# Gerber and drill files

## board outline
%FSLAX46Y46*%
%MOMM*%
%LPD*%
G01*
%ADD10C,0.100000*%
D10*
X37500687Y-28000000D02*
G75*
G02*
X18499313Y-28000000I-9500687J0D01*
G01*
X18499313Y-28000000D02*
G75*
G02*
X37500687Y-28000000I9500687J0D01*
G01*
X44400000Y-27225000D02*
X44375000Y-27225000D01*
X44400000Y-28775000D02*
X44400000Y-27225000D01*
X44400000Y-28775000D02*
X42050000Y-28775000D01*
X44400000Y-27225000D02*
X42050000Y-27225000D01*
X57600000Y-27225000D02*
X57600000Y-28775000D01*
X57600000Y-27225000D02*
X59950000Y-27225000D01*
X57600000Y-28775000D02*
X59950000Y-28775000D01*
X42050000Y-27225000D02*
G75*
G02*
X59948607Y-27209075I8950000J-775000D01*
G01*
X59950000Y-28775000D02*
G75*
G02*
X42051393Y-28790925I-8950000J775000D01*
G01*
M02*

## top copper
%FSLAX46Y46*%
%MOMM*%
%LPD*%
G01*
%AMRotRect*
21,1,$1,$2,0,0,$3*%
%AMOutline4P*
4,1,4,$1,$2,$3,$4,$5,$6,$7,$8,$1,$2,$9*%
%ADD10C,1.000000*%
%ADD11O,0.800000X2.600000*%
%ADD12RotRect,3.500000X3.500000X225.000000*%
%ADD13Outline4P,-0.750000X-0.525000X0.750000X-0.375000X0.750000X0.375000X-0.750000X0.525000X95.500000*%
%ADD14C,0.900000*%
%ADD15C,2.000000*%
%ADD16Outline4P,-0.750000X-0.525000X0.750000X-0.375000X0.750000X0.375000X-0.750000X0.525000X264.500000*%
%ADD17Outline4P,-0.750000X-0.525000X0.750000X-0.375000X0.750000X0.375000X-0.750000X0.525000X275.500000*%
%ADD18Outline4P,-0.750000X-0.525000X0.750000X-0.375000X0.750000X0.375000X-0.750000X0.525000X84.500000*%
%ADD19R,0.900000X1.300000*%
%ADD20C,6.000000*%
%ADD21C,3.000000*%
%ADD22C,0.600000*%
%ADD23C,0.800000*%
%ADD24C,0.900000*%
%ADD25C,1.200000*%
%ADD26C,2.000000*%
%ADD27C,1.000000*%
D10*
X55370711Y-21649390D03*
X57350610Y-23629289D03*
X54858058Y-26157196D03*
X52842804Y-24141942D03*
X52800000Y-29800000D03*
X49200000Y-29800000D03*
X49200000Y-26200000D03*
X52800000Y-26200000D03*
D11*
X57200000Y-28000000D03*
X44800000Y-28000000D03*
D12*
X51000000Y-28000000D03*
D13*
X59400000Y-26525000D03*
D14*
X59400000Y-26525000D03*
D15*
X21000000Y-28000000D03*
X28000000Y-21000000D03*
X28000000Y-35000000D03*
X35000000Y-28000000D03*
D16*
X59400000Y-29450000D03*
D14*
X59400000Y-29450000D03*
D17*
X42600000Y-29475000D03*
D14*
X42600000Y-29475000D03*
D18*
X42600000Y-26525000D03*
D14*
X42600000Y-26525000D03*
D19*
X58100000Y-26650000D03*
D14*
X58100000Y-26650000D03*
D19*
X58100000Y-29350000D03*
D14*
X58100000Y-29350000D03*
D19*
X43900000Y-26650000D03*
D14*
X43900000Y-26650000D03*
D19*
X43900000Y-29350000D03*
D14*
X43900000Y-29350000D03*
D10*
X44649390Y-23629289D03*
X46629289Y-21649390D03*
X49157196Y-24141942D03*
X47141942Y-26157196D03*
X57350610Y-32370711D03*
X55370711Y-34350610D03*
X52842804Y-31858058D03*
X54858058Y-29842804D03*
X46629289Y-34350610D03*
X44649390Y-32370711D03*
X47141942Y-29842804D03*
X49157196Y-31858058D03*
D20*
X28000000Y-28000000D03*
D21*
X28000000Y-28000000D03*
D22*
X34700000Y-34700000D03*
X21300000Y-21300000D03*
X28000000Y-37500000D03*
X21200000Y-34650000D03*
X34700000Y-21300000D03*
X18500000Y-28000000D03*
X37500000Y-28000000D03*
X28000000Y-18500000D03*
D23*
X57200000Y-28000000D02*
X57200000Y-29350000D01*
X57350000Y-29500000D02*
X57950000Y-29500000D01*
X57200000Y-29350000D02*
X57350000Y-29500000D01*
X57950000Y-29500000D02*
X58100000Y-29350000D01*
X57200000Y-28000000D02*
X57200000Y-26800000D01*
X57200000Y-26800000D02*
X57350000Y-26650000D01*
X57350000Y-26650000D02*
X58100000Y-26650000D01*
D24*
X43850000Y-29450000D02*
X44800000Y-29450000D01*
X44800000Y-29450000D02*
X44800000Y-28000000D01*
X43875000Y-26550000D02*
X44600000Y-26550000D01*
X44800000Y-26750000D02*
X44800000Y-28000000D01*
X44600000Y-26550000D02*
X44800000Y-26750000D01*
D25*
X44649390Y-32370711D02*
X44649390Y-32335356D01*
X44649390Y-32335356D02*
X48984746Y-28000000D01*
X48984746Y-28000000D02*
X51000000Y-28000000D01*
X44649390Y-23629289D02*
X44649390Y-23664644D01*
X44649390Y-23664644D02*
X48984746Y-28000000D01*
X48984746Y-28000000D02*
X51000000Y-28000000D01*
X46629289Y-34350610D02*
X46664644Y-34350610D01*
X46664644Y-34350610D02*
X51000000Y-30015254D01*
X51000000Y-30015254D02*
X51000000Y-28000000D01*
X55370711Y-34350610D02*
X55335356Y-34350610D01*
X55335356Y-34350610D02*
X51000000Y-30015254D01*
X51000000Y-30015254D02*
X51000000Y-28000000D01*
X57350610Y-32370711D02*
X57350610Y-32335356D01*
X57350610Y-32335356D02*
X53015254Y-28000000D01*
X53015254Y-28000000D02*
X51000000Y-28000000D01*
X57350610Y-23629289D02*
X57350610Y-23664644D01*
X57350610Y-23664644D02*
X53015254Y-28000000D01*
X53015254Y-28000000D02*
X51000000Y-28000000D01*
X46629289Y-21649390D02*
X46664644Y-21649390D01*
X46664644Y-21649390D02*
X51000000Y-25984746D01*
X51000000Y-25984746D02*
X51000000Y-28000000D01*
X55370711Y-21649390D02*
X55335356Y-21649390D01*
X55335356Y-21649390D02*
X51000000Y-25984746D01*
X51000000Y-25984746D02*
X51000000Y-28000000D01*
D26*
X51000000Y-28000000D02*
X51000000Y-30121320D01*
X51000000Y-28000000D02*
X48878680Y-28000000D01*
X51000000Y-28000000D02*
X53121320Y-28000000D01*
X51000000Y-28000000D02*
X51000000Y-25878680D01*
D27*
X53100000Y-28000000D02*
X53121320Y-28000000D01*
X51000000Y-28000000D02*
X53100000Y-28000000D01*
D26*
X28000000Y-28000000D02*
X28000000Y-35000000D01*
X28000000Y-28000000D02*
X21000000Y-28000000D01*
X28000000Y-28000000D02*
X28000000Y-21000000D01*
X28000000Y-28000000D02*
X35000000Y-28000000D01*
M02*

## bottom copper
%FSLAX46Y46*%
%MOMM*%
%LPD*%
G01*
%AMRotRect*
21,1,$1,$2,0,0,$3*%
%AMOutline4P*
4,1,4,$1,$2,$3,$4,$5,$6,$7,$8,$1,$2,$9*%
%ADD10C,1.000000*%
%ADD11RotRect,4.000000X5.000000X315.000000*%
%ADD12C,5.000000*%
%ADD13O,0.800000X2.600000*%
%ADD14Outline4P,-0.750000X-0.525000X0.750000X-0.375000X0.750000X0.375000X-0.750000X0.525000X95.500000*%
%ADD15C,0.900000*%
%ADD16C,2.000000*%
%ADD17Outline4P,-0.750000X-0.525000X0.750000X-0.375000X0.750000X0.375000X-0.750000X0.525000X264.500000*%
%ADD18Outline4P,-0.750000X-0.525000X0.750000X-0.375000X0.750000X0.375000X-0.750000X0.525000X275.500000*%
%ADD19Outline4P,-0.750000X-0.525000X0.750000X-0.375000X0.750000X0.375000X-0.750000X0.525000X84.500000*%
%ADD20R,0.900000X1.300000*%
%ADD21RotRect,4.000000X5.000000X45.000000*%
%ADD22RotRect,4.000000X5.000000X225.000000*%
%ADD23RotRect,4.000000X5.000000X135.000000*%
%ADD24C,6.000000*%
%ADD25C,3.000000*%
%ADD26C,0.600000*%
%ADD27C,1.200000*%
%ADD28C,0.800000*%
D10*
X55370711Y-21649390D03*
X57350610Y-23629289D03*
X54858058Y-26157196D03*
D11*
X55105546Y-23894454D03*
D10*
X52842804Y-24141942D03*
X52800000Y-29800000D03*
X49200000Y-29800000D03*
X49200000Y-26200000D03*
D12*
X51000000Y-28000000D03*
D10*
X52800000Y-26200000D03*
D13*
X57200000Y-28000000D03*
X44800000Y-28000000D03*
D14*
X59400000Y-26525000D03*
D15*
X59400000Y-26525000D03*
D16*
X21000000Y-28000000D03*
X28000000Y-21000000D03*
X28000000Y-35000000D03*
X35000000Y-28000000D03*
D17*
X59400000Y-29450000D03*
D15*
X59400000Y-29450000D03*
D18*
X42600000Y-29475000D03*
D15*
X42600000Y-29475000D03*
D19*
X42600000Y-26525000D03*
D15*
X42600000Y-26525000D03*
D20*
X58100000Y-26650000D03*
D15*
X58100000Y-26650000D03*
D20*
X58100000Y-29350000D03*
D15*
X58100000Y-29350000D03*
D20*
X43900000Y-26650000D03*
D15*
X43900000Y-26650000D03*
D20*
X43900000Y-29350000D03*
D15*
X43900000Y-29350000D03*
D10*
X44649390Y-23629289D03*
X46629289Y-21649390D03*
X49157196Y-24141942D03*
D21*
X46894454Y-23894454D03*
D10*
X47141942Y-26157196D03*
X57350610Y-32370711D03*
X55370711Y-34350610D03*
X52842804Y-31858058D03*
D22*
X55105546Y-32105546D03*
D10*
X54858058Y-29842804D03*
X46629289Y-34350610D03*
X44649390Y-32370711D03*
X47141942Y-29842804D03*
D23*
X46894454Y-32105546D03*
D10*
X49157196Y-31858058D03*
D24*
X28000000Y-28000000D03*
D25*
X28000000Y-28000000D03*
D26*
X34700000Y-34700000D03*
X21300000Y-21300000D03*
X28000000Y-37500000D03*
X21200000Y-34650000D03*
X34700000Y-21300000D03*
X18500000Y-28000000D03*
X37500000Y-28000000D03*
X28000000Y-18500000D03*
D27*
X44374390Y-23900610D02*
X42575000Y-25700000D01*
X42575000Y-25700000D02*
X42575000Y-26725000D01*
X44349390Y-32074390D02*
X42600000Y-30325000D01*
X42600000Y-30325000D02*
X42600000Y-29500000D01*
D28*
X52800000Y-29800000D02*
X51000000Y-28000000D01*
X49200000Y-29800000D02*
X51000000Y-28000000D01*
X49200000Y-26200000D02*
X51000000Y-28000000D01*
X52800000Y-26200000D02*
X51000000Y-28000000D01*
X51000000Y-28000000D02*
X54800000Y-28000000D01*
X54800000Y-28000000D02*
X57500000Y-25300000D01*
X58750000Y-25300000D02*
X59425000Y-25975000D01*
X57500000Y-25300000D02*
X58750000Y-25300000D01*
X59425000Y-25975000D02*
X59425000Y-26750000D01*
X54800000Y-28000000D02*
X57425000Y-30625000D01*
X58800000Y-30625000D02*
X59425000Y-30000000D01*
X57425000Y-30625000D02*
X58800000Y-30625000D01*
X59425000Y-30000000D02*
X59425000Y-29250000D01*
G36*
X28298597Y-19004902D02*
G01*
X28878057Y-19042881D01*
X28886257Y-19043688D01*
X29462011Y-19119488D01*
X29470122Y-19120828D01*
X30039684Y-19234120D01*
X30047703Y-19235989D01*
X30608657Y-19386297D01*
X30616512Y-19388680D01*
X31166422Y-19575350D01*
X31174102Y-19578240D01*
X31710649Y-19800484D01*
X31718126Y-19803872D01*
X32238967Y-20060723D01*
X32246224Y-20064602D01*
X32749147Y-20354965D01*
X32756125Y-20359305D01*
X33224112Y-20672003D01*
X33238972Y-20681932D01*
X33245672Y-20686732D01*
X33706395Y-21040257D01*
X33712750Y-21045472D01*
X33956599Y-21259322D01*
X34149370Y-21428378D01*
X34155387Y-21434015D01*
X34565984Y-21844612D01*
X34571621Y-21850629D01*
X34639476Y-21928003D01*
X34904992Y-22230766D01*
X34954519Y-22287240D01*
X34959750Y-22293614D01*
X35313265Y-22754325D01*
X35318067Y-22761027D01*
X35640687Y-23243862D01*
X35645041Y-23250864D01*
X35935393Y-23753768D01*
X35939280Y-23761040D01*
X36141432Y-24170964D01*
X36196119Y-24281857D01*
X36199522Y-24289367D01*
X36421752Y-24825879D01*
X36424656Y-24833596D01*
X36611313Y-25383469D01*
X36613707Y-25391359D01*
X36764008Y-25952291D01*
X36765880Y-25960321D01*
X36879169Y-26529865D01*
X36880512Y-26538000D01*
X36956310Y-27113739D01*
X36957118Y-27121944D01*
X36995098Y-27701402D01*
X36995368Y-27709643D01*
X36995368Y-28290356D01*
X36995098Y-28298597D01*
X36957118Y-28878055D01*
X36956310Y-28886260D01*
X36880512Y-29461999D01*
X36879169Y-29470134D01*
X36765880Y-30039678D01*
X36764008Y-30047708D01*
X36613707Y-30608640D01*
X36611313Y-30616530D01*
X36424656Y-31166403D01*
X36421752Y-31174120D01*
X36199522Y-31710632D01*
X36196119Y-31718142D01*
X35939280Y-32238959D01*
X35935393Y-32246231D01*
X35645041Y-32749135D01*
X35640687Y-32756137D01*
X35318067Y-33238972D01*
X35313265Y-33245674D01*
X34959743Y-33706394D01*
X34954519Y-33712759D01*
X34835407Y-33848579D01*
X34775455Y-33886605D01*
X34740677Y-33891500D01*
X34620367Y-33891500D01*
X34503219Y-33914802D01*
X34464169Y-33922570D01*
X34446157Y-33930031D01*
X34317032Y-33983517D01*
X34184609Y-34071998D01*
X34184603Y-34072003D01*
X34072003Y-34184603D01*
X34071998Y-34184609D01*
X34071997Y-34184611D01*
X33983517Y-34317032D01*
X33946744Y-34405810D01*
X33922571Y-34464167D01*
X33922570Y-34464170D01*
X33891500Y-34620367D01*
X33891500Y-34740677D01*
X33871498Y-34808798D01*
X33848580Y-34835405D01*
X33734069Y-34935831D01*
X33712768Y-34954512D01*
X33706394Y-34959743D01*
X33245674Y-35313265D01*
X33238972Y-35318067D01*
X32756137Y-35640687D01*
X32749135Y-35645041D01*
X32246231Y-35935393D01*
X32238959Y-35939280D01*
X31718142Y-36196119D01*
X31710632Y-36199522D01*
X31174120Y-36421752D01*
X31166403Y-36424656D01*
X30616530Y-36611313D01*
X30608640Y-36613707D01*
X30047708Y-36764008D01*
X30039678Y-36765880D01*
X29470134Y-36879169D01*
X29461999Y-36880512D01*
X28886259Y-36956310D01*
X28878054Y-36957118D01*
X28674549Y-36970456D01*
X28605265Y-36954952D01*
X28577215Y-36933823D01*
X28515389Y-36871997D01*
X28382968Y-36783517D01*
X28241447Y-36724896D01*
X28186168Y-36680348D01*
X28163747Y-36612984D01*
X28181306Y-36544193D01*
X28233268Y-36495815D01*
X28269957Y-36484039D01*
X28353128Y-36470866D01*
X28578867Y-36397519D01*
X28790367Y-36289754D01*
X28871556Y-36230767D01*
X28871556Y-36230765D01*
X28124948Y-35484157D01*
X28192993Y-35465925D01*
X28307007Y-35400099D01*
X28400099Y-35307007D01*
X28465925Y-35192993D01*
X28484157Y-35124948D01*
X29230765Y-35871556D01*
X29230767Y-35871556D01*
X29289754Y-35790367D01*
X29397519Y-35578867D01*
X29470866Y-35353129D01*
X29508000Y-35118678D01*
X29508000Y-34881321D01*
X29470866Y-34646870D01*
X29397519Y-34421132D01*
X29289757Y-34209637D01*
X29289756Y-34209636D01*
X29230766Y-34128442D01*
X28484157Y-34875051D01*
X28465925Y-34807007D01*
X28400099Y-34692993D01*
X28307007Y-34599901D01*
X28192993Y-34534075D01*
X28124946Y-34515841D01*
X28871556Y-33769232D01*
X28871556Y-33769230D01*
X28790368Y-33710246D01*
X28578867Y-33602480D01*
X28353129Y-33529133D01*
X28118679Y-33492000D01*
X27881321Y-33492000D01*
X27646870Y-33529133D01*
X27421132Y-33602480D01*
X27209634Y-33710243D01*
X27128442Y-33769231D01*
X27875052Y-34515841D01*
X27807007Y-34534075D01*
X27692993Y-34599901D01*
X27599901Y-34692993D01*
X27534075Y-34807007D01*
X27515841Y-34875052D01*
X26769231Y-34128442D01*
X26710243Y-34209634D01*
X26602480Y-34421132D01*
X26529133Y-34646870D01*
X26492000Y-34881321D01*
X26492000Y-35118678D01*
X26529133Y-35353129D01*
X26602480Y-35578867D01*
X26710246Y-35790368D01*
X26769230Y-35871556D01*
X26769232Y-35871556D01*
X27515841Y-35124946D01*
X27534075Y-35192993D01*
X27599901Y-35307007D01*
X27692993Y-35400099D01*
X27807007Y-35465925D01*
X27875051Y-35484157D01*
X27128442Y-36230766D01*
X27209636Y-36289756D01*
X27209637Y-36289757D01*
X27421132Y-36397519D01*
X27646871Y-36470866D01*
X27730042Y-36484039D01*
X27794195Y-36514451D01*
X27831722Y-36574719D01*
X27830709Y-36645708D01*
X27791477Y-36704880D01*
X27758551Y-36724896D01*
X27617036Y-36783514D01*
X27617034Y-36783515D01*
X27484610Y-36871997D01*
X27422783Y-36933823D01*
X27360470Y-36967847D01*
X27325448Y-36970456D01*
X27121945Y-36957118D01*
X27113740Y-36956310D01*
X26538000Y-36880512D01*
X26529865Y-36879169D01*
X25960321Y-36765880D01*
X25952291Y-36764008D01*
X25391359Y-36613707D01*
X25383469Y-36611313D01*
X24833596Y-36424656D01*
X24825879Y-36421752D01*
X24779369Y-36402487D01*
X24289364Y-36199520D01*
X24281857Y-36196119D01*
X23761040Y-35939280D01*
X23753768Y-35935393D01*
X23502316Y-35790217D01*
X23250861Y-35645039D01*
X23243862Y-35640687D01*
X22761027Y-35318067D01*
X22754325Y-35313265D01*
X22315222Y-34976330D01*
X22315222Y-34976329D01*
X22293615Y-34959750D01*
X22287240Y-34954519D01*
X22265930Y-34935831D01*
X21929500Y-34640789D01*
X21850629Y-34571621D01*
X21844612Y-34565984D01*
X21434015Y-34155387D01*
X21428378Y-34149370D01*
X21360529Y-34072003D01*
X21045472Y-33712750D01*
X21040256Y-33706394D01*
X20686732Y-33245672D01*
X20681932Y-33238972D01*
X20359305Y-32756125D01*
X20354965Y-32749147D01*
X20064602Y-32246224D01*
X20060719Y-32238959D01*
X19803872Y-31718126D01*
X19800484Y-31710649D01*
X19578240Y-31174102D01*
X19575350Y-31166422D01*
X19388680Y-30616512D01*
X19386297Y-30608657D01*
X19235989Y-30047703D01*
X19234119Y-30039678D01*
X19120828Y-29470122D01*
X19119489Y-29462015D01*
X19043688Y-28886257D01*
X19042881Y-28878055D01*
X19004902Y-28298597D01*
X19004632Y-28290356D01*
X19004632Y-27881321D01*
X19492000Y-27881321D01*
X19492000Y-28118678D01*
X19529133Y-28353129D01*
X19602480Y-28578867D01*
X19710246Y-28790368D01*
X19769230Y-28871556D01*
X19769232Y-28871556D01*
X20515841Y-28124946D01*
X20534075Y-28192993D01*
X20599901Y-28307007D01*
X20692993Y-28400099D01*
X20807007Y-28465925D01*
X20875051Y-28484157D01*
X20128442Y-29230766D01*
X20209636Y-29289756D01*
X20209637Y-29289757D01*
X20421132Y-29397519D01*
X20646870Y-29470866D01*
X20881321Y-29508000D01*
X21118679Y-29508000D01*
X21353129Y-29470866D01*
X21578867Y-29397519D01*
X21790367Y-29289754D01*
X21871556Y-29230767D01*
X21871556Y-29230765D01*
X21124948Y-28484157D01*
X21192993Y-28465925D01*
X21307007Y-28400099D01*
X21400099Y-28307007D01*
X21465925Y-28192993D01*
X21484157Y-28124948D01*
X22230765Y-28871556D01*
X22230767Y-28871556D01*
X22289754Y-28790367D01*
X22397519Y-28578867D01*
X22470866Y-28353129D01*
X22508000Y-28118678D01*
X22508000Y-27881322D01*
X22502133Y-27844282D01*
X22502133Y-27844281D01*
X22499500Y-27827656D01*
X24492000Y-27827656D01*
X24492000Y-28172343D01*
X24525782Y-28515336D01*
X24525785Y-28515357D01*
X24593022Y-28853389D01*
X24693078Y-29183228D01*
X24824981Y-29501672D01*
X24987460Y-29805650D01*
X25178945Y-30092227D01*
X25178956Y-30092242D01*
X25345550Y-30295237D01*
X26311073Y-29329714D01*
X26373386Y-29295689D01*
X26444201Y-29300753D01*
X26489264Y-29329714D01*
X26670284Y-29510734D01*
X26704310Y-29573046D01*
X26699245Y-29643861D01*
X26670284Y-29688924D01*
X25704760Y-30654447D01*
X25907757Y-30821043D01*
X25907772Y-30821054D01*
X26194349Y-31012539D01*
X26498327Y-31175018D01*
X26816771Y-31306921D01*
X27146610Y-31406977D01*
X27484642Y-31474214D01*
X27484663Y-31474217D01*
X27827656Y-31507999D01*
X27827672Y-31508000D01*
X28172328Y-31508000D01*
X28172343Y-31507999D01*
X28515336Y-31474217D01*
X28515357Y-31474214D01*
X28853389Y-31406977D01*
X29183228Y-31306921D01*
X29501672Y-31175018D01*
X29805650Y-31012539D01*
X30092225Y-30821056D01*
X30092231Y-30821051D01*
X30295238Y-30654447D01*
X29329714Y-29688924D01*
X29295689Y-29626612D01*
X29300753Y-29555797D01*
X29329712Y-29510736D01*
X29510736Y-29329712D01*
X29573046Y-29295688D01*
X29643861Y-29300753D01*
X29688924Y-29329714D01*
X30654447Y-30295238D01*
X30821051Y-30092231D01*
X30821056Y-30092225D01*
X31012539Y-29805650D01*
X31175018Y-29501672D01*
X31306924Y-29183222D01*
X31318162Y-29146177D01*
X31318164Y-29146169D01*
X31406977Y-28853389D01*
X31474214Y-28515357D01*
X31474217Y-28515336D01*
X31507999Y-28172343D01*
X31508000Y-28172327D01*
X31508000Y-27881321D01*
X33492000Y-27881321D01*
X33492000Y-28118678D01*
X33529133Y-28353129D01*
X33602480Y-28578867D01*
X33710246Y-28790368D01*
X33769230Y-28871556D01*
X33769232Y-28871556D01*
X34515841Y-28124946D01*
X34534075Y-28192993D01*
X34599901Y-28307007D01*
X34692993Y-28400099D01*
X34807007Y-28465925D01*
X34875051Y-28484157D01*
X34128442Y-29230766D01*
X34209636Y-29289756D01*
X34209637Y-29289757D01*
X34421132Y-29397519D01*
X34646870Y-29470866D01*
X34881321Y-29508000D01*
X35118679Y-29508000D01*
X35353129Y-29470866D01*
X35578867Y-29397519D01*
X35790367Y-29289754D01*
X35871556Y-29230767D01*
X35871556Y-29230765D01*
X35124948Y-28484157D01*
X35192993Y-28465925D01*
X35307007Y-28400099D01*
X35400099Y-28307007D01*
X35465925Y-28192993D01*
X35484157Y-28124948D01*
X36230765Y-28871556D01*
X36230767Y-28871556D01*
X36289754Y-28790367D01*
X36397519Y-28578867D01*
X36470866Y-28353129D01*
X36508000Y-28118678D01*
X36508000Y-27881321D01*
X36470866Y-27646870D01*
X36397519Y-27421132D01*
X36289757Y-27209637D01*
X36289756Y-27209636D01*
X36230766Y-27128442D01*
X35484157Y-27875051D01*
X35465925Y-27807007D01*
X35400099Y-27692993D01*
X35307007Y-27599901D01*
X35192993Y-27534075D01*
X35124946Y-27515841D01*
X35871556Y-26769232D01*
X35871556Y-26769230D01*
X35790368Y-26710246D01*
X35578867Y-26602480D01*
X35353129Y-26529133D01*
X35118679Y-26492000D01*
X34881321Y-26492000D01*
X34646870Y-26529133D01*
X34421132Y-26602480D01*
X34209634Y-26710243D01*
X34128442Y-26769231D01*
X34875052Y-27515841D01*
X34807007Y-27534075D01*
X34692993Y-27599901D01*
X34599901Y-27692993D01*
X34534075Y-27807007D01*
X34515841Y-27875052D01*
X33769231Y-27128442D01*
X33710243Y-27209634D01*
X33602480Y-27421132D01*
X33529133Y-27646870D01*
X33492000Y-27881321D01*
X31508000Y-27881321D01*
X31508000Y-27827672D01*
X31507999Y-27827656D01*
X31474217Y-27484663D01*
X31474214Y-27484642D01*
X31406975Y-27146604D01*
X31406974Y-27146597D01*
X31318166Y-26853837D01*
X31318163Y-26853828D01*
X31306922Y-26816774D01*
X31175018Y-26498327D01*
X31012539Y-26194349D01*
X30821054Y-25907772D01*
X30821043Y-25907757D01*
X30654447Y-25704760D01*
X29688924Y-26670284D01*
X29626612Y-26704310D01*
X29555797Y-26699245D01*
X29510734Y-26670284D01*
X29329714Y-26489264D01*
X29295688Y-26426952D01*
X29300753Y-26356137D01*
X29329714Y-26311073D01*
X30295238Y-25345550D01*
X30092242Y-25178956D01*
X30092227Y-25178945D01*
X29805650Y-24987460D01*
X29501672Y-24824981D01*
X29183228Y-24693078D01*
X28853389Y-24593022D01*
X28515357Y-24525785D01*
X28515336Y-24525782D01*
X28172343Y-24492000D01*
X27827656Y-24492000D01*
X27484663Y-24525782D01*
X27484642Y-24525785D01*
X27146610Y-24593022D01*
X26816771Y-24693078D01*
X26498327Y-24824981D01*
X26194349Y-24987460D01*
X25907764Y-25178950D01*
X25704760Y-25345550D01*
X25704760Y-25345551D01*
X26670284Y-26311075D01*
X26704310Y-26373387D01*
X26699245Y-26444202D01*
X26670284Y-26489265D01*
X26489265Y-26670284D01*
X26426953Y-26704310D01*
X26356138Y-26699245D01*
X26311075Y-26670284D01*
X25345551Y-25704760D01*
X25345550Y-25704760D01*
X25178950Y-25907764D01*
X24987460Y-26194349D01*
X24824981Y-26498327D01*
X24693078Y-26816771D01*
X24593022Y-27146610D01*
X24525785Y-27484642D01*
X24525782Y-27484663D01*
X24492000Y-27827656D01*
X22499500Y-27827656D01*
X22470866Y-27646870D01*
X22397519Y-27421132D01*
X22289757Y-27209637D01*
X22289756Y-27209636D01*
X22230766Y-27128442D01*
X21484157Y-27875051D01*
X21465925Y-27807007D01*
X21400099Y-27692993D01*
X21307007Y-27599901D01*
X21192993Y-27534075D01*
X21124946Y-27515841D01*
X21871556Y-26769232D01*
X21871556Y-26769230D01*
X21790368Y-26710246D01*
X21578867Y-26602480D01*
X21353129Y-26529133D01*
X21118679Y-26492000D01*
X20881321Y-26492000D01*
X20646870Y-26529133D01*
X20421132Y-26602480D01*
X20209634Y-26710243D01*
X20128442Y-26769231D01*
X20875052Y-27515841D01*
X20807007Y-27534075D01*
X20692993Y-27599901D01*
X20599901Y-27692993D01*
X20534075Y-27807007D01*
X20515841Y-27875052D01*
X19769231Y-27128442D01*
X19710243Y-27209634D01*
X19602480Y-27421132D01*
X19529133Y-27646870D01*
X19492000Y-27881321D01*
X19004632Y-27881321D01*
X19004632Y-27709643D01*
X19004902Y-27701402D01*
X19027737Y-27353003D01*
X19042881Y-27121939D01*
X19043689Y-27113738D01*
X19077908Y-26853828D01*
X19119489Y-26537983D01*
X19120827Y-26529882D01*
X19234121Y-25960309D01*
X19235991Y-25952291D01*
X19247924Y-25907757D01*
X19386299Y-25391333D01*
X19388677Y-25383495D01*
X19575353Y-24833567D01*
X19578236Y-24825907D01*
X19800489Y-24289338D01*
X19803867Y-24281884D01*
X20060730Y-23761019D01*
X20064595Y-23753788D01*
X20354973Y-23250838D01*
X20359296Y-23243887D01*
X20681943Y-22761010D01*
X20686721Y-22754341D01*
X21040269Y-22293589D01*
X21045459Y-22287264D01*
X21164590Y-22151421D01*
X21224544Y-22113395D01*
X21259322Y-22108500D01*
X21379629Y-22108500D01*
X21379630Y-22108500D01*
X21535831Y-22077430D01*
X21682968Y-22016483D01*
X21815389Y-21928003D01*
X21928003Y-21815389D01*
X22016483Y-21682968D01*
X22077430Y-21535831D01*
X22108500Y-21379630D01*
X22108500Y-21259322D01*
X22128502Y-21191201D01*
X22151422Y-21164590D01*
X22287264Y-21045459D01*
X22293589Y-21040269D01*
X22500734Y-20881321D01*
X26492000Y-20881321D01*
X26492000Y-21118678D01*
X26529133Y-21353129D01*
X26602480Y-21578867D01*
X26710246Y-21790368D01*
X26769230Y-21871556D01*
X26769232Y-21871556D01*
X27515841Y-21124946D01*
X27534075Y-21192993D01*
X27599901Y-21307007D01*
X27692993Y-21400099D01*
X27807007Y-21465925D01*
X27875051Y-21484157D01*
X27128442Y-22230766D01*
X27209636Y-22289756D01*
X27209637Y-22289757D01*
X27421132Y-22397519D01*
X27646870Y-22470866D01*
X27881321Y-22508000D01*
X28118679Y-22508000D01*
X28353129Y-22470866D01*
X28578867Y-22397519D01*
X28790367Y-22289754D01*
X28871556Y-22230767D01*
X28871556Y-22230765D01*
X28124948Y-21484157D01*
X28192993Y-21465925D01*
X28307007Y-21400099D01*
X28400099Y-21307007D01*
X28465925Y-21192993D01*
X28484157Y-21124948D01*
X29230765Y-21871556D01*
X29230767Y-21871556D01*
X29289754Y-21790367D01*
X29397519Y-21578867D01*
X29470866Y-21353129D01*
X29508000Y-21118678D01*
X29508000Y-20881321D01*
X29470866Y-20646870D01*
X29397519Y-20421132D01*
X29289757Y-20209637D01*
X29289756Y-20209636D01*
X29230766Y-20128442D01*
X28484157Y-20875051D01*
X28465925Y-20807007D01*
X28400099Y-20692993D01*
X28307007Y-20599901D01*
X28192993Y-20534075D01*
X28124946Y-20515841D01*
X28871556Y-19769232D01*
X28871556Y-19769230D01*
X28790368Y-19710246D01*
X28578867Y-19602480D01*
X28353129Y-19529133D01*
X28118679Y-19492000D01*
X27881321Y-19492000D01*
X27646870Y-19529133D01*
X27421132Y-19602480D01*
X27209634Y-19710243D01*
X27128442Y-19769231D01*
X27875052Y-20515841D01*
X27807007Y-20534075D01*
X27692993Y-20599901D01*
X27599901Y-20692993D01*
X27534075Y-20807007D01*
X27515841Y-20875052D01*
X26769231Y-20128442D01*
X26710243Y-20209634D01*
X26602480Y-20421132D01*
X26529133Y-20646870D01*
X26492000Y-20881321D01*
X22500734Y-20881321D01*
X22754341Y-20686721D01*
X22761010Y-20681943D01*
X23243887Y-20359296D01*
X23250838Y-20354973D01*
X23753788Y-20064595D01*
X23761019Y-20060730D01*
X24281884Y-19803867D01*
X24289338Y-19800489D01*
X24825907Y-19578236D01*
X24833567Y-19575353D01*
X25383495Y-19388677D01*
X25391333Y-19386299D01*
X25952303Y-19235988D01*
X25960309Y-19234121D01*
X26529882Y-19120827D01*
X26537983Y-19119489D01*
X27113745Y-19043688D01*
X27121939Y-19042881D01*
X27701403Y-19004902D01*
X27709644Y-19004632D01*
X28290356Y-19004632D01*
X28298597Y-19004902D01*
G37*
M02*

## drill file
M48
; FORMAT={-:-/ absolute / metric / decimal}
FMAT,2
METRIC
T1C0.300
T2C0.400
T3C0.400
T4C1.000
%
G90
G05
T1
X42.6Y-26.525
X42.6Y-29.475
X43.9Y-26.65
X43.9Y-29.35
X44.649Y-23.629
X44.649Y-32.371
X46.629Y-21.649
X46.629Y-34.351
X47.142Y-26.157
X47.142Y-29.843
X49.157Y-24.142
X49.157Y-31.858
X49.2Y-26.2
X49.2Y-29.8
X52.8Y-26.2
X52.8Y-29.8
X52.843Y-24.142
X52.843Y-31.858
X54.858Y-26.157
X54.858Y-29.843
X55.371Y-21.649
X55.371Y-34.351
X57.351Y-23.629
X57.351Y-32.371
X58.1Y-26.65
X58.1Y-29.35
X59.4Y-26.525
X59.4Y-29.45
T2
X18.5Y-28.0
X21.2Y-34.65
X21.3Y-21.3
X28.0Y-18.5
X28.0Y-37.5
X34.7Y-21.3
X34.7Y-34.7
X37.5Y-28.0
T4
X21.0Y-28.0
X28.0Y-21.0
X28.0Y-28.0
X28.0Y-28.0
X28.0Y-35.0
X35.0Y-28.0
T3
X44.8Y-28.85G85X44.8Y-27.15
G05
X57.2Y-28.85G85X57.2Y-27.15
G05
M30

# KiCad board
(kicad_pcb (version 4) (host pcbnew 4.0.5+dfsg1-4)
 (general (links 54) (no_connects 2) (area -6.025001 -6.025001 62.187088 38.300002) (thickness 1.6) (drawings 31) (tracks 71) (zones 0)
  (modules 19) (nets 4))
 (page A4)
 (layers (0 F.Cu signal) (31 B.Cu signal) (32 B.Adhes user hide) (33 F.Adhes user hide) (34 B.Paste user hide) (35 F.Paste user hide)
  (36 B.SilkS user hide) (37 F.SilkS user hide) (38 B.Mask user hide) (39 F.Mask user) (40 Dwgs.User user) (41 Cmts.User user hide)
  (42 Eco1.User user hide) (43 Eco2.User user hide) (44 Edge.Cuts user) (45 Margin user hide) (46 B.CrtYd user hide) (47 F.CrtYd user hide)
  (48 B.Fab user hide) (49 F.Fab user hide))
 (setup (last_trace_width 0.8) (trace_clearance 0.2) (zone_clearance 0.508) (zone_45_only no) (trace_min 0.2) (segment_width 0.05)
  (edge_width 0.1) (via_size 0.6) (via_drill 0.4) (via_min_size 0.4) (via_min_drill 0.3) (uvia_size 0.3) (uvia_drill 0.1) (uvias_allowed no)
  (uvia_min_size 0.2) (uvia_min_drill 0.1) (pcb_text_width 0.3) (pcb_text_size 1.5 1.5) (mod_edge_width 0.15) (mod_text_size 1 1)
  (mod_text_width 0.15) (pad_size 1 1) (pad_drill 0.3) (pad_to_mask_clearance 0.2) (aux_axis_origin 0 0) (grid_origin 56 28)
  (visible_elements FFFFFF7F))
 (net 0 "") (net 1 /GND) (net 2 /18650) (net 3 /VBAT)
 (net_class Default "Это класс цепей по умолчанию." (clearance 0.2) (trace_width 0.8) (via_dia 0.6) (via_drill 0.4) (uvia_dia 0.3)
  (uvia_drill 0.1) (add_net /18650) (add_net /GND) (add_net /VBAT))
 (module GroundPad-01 (layer F.Cu) (at 55.3 23.7 315)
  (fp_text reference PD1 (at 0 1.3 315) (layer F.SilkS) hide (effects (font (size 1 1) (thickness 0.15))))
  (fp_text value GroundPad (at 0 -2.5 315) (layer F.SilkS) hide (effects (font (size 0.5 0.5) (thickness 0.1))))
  (pad 2 thru_hole circle (at -1.4 -1.5 315) (size 1 1) (drill 0.3) (layers *.Cu) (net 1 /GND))
  (pad 3 thru_hole circle (at 1.4 -1.5 315) (size 1 1) (drill 0.3) (layers *.Cu) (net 1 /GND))
  (pad 5 thru_hole circle (at 1.425 2.05 315) (size 1 1) (drill 0.3) (layers *.Cu) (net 1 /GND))
  (pad 1 smd rect (at 0 0.275 315) (size 4 5) (layers B.Cu B.Paste B.Mask) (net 1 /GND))
  (pad 4 thru_hole circle (at -1.425 2.05 315) (size 1 1) (drill 0.3) (layers *.Cu) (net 1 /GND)))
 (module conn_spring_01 (layer B.Cu) (at 51 28 270)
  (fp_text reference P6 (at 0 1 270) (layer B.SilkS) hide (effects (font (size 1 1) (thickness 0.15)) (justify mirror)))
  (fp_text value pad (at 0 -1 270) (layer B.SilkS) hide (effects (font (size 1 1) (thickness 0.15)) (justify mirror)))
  (pad 4 thru_hole circle (at 1.8 -1.8 270) (size 1 1) (drill 0.3) (layers *.Cu) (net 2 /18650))
  (pad 3 thru_hole circle (at 1.8 1.8 270) (size 1 1) (drill 0.3) (layers *.Cu) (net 2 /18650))
  (pad 2 thru_hole circle (at -1.8 1.8 270) (size 1 1) (drill 0.3) (layers *.Cu) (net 2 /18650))
  (pad 1 smd circle (at 0 0 270) (size 5 5) (layers B.Cu B.Paste B.Mask) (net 2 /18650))
  (pad 5 thru_hole circle (at -1.8 -1.8 270) (size 1 1) (drill 0.3) (layers *.Cu) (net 2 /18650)))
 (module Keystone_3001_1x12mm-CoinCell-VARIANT (layer F.Cu) (at 51 28 180)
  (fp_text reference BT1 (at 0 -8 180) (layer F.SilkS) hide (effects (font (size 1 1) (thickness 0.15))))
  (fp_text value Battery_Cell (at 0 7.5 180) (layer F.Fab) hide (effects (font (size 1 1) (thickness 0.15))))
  (pad 1 thru_hole oval (at -6.2 0 180) (size 0.8 2.6) (drill oval 0.4 2.1) (layers *.Cu *.Mask) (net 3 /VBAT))
  (pad 1 thru_hole oval (at 6.2 0 180) (size 0.8 2.6) (drill oval 0.4 2.1) (layers *.Cu *.Mask) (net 3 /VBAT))
  (pad 2 smd rect (at 0 0 225) (size 3.5 3.5) (layers F.Cu F.Mask) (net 1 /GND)))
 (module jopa (layer F.Cu) (at 59.4 26.525 95.5)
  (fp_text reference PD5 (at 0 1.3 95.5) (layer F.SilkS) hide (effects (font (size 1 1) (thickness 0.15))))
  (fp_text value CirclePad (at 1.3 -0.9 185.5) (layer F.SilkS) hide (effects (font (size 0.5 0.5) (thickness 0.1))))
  (pad 1 smd trapezoid (at 0 0 95.5) (size 1.5 0.9) (rect_delta 0.15 0) (layers F.Cu F.Paste F.Mask) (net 2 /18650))
  (pad 2 smd trapezoid (at 0 0 95.5) (size 1.5 0.9) (rect_delta 0.15 0) (layers B.Cu F.Paste B.Mask) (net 2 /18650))
  (pad 3 thru_hole circle (at 0 0 95.5) (size 0.9 0.9) (drill 0.3) (layers *.Cu *.Mask) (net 2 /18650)))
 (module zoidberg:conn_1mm (layer F.Cu) (at 21 28)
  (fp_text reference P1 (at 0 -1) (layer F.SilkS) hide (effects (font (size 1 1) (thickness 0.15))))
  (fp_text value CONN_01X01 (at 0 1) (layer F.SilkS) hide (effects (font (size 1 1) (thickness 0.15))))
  (pad 1 thru_hole circle (at 0 0) (size 2 2) (drill 1) (layers *.Cu) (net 1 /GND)))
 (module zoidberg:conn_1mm (layer F.Cu) (at 28 21)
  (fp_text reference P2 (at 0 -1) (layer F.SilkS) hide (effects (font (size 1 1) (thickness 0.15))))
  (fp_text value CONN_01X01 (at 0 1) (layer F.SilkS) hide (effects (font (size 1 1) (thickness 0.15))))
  (pad 1 thru_hole circle (at 0 0) (size 2 2) (drill 1) (layers *.Cu) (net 1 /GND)))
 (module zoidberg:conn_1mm (layer F.Cu) (at 28 35)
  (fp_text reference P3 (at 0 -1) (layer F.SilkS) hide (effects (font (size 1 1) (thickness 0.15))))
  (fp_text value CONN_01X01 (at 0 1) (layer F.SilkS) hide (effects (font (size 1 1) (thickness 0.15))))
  (pad 1 thru_hole circle (at 0 0) (size 2 2) (drill 1) (layers *.Cu) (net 1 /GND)))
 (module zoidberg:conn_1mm (layer F.Cu) (at 35 28)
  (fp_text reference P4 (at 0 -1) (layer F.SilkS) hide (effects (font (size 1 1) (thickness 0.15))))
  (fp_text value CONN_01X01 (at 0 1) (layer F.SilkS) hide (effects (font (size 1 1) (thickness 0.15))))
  (pad 1 thru_hole circle (at 0 0) (size 2 2) (drill 1) (layers *.Cu) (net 1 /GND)))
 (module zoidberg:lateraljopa (layer F.Cu) (at 59.4 29.45 264.5)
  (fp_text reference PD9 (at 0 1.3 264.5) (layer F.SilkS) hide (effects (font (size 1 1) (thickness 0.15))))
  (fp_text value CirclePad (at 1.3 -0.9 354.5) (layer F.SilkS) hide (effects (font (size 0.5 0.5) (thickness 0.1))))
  (pad 1 smd trapezoid (at 0 0 264.5) (size 1.5 0.9) (rect_delta 0.15 0) (layers F.Cu F.Paste F.Mask) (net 2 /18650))
  (pad 2 smd trapezoid (at 0 0 264.5) (size 1.5 0.9) (rect_delta 0.15 0) (layers B.Cu F.Paste B.Mask) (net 2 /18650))
  (pad 3 thru_hole circle (at 0 0 264.5) (size 0.9 0.9) (drill 0.3) (layers *.Cu *.Mask) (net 2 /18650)))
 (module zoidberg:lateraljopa (layer F.Cu) (at 42.6 29.475 275.5)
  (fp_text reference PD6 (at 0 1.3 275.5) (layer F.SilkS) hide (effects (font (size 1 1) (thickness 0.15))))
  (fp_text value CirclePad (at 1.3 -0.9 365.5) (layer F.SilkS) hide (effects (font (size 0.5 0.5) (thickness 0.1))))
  (pad 1 smd trapezoid (at 0 0 275.5) (size 1.5 0.9) (rect_delta 0.15 0) (layers F.Cu F.Paste F.Mask) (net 1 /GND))
  (pad 2 smd trapezoid (at 0 0 275.5) (size 1.5 0.9) (rect_delta 0.15 0) (layers B.Cu F.Paste B.Mask) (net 1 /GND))
  (pad 3 thru_hole circle (at 0 0 275.5) (size 0.9 0.9) (drill 0.3) (layers *.Cu *.Mask) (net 1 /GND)))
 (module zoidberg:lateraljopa (layer F.Cu) (at 42.6 26.525 84.5)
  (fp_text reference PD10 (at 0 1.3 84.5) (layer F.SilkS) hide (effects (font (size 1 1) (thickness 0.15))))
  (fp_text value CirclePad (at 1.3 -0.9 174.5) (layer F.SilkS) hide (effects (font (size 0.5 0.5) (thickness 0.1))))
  (pad 1 smd trapezoid (at 0 0 84.5) (size 1.5 0.9) (rect_delta 0.15 0) (layers F.Cu F.Paste F.Mask) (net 1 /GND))
  (pad 2 smd trapezoid (at 0 0 84.5) (size 1.5 0.9) (rect_delta 0.15 0) (layers B.Cu F.Paste B.Mask) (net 1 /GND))
  (pad 3 thru_hole circle (at 0 0 84.5) (size 0.9 0.9) (drill 0.3) (layers *.Cu *.Mask) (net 1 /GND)))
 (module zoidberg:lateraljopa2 (layer F.Cu) (at 58.1 26.65 90)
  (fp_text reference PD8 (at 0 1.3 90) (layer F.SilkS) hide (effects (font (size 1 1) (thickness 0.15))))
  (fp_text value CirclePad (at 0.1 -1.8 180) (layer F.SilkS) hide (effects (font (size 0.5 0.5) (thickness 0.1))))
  (pad 1 smd rect (at 0 0 90) (size 1.3 0.9) (layers F.Cu F.Paste F.Mask) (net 3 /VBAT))
  (pad 2 smd rect (at 0 0 90) (size 1.3 0.9) (layers B.Cu F.Paste B.Mask) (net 3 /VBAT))
  (pad 3 thru_hole circle (at 0 0 90) (size 0.9 0.9) (drill 0.3) (layers *.Cu *.Mask) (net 3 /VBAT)))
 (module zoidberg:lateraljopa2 (layer F.Cu) (at 58.1 29.35 90)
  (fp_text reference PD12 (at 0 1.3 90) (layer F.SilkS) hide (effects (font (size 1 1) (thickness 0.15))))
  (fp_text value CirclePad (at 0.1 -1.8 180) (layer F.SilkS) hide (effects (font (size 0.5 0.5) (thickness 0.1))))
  (pad 1 smd rect (at 0 0 90) (size 1.3 0.9) (layers F.Cu F.Paste F.Mask) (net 3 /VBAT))
  (pad 2 smd rect (at 0 0 90) (size 1.3 0.9) (layers B.Cu F.Paste B.Mask) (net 3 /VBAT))
  (pad 3 thru_hole circle (at 0 0 90) (size 0.9 0.9) (drill 0.3) (layers *.Cu *.Mask) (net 3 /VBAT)))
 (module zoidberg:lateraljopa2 (layer F.Cu) (at 43.9 26.65 90)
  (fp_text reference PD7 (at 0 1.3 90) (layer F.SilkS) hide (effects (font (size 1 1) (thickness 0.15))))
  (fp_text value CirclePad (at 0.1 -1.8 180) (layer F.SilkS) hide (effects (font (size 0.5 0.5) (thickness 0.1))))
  (pad 1 smd rect (at 0 0 90) (size 1.3 0.9) (layers F.Cu F.Paste F.Mask) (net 3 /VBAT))
  (pad 2 smd rect (at 0 0 90) (size 1.3 0.9) (layers B.Cu F.Paste B.Mask) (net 3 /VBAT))
  (pad 3 thru_hole circle (at 0 0 90) (size 0.9 0.9) (drill 0.3) (layers *.Cu *.Mask) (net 3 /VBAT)))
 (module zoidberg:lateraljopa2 (layer F.Cu) (at 43.9 29.35 90)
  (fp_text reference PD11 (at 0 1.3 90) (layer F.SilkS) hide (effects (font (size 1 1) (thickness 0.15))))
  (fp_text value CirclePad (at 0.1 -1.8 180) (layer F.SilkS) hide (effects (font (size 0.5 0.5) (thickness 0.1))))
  (pad 1 smd rect (at 0 0 90) (size 1.3 0.9) (layers F.Cu F.Paste F.Mask) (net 3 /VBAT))
  (pad 2 smd rect (at 0 0 90) (size 1.3 0.9) (layers B.Cu F.Paste B.Mask) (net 3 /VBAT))
  (pad 3 thru_hole circle (at 0 0 90) (size 0.9 0.9) (drill 0.3) (layers *.Cu *.Mask) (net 3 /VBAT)))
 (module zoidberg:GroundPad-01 (layer F.Cu) (at 46.7 23.7 45)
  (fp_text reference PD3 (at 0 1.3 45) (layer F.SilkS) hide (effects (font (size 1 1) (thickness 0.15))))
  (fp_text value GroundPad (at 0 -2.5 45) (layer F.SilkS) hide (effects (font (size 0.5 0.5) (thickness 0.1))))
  (pad 2 thru_hole circle (at -1.4 -1.5 45) (size 1 1) (drill 0.3) (layers *.Cu) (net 1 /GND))
  (pad 3 thru_hole circle (at 1.4 -1.5 45) (size 1 1) (drill 0.3) (layers *.Cu) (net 1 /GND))
  (pad 5 thru_hole circle (at 1.425 2.05 45) (size 1 1) (drill 0.3) (layers *.Cu) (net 1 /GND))
  (pad 1 smd rect (at 0 0.275 45) (size 4 5) (layers B.Cu B.Paste B.Mask) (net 1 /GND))
  (pad 4 thru_hole circle (at -1.425 2.05 45) (size 1 1) (drill 0.3) (layers *.Cu) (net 1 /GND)))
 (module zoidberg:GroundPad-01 (layer F.Cu) (at 55.3 32.3 225)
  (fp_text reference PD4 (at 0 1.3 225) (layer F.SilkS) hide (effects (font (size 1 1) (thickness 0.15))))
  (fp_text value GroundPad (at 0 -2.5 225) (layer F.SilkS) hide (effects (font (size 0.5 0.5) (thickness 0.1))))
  (pad 2 thru_hole circle (at -1.4 -1.5 225) (size 1 1) (drill 0.3) (layers *.Cu) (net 1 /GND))
  (pad 3 thru_hole circle (at 1.4 -1.5 225) (size 1 1) (drill 0.3) (layers *.Cu) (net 1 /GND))
  (pad 5 thru_hole circle (at 1.425 2.05 225) (size 1 1) (drill 0.3) (layers *.Cu) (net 1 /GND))
  (pad 1 smd rect (at 0 0.275 225) (size 4 5) (layers B.Cu B.Paste B.Mask) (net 1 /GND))
  (pad 4 thru_hole circle (at -1.425 2.05 225) (size 1 1) (drill 0.3) (layers *.Cu) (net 1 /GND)))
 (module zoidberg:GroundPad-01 (layer F.Cu) (at 46.7 32.3 135)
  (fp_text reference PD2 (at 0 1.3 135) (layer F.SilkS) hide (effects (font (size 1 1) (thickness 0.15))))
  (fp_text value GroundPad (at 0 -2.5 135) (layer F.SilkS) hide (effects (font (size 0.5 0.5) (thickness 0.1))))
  (pad 2 thru_hole circle (at -1.4 -1.5 135) (size 1 1) (drill 0.3) (layers *.Cu) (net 1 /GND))
  (pad 3 thru_hole circle (at 1.4 -1.5 135) (size 1 1) (drill 0.3) (layers *.Cu) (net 1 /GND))
  (pad 5 thru_hole circle (at 1.425 2.05 135) (size 1 1) (drill 0.3) (layers *.Cu) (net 1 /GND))
  (pad 1 smd rect (at 0 0.275 135) (size 4 5) (layers B.Cu B.Paste B.Mask) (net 1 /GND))
  (pad 4 thru_hole circle (at -1.425 2.05 135) (size 1 1) (drill 0.3) (layers *.Cu) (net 1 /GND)))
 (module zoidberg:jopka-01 (layer F.Cu) (at 28 28)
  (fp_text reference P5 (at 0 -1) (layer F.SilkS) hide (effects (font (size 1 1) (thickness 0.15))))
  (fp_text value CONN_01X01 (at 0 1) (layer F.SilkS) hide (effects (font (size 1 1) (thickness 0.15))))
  (pad 1 thru_hole circle (at 0 0) (size 6 6) (drill 1) (layers *.Cu *.Mask) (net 1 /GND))
  (pad 2 thru_hole circle (at 0 0) (size 3 3) (drill 1) (layers *.Mask B.Cu)))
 (gr_circle (center 28 28) (end 34.718 34.718) (layer Edge.Cuts) (width 0.1))
 (gr_line (start 44.4 27.225) (end 44.375 27.225) (angle 90) (layer Edge.Cuts) (width 0.1))
 (gr_line (start 44.4 28.775) (end 44.4 27.225) (angle 90) (layer Edge.Cuts) (width 0.1))
 (gr_line (start 44.4 28.775) (end 42.05 28.775) (angle 90) (layer Edge.Cuts) (width 0.1))
 (gr_line (start 44.4 27.225) (end 42.05 27.225) (angle 90) (layer Edge.Cuts) (width 0.1))
 (gr_line (start 57.6 27.225) (end 57.6 28.775) (angle 90) (layer Edge.Cuts) (width 0.1))
 (gr_line (start 57.6 27.225) (end 59.95 27.225) (angle 90) (layer Edge.Cuts) (width 0.1))
 (gr_line (start 57.6 28.775) (end 59.95 28.775) (angle 90) (layer Edge.Cuts) (width 0.1))
 (gr_arc (start 51 28) (end 42.05 27.225) (angle 170) (layer Edge.Cuts) (width 0.1))
 (gr_arc (start 51 28) (end 59.95 28.775) (angle 170) (layer Edge.Cuts) (width 0.1))
 (via (at 34.7 34.7) (size 0.6) (drill 0.4) (layers F.Cu B.Cu) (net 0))
 (via (at 21.3 21.3) (size 0.6) (drill 0.4) (layers F.Cu B.Cu) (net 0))
 (via (at 28 37.5) (size 0.6) (drill 0.4) (layers F.Cu B.Cu) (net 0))
 (segment (start 57.2 28) (end 57.2 29.35) (width 0.8) (layer F.Cu) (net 3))
 (segment (start 57.35 29.5) (end 57.95 29.5) (width 0.8) (layer F.Cu) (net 3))
 (segment (start 57.2 29.35) (end 57.35 29.5) (width 0.8) (layer F.Cu) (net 3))
 (segment (start 57.95 29.5) (end 58.1 29.35) (width 0.8) (layer F.Cu) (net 3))
 (segment (start 57.2 28) (end 57.2 26.8) (width 0.8) (layer F.Cu) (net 3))
 (segment (start 57.2 26.8) (end 57.35 26.65) (width 0.8) (layer F.Cu) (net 3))
 (segment (start 57.35 26.65) (end 58.1 26.65) (width 0.8) (layer F.Cu) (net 3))
 (segment (start 43.85 29.45) (end 44.8 29.45) (width 0.9) (layer F.Cu) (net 3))
 (segment (start 44.8 29.45) (end 44.8 28) (width 0.9) (layer F.Cu) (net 3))
 (segment (start 43.875 26.55) (end 44.6 26.55) (width 0.9) (layer F.Cu) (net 3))
 (segment (start 44.8 26.75) (end 44.8 28) (width 0.9) (layer F.Cu) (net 3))
 (segment (start 44.6 26.55) (end 44.8 26.75) (width 0.9) (layer F.Cu) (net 3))
 (via (at 21.2 34.65) (size 0.6) (drill 0.4) (layers F.Cu B.Cu) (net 1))
 (via (at 34.7 21.3) (size 0.6) (drill 0.4) (layers F.Cu B.Cu) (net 1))
 (via (at 18.5 28) (size 0.6) (drill 0.4) (layers F.Cu B.Cu) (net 1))
 (via (at 37.5 28) (size 0.6) (drill 0.4) (layers F.Cu B.Cu) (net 1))
 (via (at 28 18.5) (size 0.6) (drill 0.4) (layers F.Cu B.Cu) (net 1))
 (segment (start 44.64939 32.370711) (end 44.64939 32.335356) (width 1.2) (layer F.Cu) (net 1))
 (segment (start 44.64939 32.335356) (end 48.984746 28) (width 1.2) (layer F.Cu) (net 1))
 (segment (start 48.984746 28) (end 51 28) (width 1.2) (layer F.Cu) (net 1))
 (segment (start 44.64939 23.629289) (end 44.64939 23.664644) (width 1.2) (layer F.Cu) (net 1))
 (segment (start 44.64939 23.664644) (end 48.984746 28) (width 1.2) (layer F.Cu) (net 1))
 (segment (start 48.984746 28) (end 51 28) (width 1.2) (layer F.Cu) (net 1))
 (segment (start 46.629289 34.35061) (end 46.664644 34.35061) (width 1.2) (layer F.Cu) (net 1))
 (segment (start 46.664644 34.35061) (end 51 30.015254) (width 1.2) (layer F.Cu) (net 1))
 (segment (start 51 30.015254) (end 51 28) (width 1.2) (layer F.Cu) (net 1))
 (segment (start 55.370711 34.35061) (end 55.335356 34.35061) (width 1.2) (layer F.Cu) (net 1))
 (segment (start 55.335356 34.35061) (end 51 30.015254) (width 1.2) (layer F.Cu) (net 1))
 (segment (start 51 30.015254) (end 51 28) (width 1.2) (layer F.Cu) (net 1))
 (segment (start 57.35061 32.370711) (end 57.35061 32.335356) (width 1.2) (layer F.Cu) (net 1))
 (segment (start 57.35061 32.335356) (end 53.015254 28) (width 1.2) (layer F.Cu) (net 1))
 (segment (start 53.015254 28) (end 51 28) (width 1.2) (layer F.Cu) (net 1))
 (segment (start 57.35061 23.629289) (end 57.35061 23.664644) (width 1.2) (layer F.Cu) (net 1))
 (segment (start 57.35061 23.664644) (end 53.015254 28) (width 1.2) (layer F.Cu) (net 1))
 (segment (start 53.015254 28) (end 51 28) (width 1.2) (layer F.Cu) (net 1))
 (segment (start 46.629289 21.64939) (end 46.664644 21.64939) (width 1.2) (layer F.Cu) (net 1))
 (segment (start 46.664644 21.64939) (end 51 25.984746) (width 1.2) (layer F.Cu) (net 1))
 (segment (start 51 25.984746) (end 51 28) (width 1.2) (layer F.Cu) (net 1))
 (segment (start 55.370711 21.64939) (end 55.335356 21.64939) (width 1.2) (layer F.Cu) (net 1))
 (segment (start 55.335356 21.64939) (end 51 25.984746) (width 1.2) (layer F.Cu) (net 1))
 (segment (start 51 25.984746) (end 51 28) (width 1.2) (layer F.Cu) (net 1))
 (segment (start 44.37439 23.90061) (end 42.575 25.7) (width 1.2) (layer B.Cu) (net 1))
 (segment (start 42.575 25.7) (end 42.575 26.725) (width 1.2) (layer B.Cu) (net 1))
 (segment (start 44.34939 32.07439) (end 42.6 30.325) (width 1.2) (layer B.Cu) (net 1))
 (segment (start 42.6 30.325) (end 42.6 29.5) (width 1.2) (layer B.Cu) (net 1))
 (segment (start 51 28) (end 51 30.12132) (width 2) (layer F.Cu) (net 1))
 (segment (start 51 28) (end 48.87868 28) (width 2) (layer F.Cu) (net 1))
 (segment (start 51 28) (end 53.12132 28) (width 2) (layer F.Cu) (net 1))
 (segment (start 51 28) (end 51 25.87868) (width 2) (layer F.Cu) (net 1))
 (segment (start 53.1 28) (end 53.12132 28) (width 1) (layer F.Cu) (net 1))
 (segment (start 51 28) (end 53.1 28) (width 1) (layer F.Cu) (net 1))
 (segment (start 28 28) (end 28 35) (width 2) (layer F.Cu) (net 1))
 (segment (start 28 28) (end 21 28) (width 2) (layer F.Cu) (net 1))
 (segment (start 28 28) (end 28 21) (width 2) (layer F.Cu) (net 1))
 (segment (start 28 28) (end 35 28) (width 2) (layer F.Cu) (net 1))
 (segment (start 52.8 29.8) (end 51 28) (width 0.8) (layer B.Cu) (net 2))
 (segment (start 49.2 29.8) (end 51 28) (width 0.8) (layer B.Cu) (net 2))
 (segment (start 49.2 26.2) (end 51 28) (width 0.8) (layer B.Cu) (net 2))
 (segment (start 52.8 26.2) (end 51 28) (width 0.8) (layer B.Cu) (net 2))
 (segment (start 51 28) (end 54.8 28) (width 0.8) (layer B.Cu) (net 2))
 (segment (start 54.8 28) (end 57.5 25.3) (width 0.8) (layer B.Cu) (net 2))
 (segment (start 58.75 25.3) (end 59.425 25.975) (width 0.8) (layer B.Cu) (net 2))
 (segment (start 57.5 25.3) (end 58.75 25.3) (width 0.8) (layer B.Cu) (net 2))
 (segment (start 59.425 25.975) (end 59.425 26.75) (width 0.8) (layer B.Cu) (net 2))
 (segment (start 54.8 28) (end 57.425 30.625) (width 0.8) (layer B.Cu) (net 2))
 (segment (start 58.8 30.625) (end 59.425 30) (width 0.8) (layer B.Cu) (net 2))
 (segment (start 57.425 30.625) (end 58.8 30.625) (width 0.8) (layer B.Cu) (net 2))
 (segment (start 59.425 30) (end 59.425 29.25) (width 0.8) (layer B.Cu) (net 2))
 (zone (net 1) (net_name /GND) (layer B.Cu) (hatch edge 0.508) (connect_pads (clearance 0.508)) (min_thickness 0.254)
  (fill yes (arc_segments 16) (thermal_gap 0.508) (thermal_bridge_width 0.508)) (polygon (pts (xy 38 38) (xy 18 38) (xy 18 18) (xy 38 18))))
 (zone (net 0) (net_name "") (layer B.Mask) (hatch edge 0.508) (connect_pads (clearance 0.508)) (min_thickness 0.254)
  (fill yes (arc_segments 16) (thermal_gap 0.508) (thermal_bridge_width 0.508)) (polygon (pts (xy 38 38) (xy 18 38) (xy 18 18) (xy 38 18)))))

